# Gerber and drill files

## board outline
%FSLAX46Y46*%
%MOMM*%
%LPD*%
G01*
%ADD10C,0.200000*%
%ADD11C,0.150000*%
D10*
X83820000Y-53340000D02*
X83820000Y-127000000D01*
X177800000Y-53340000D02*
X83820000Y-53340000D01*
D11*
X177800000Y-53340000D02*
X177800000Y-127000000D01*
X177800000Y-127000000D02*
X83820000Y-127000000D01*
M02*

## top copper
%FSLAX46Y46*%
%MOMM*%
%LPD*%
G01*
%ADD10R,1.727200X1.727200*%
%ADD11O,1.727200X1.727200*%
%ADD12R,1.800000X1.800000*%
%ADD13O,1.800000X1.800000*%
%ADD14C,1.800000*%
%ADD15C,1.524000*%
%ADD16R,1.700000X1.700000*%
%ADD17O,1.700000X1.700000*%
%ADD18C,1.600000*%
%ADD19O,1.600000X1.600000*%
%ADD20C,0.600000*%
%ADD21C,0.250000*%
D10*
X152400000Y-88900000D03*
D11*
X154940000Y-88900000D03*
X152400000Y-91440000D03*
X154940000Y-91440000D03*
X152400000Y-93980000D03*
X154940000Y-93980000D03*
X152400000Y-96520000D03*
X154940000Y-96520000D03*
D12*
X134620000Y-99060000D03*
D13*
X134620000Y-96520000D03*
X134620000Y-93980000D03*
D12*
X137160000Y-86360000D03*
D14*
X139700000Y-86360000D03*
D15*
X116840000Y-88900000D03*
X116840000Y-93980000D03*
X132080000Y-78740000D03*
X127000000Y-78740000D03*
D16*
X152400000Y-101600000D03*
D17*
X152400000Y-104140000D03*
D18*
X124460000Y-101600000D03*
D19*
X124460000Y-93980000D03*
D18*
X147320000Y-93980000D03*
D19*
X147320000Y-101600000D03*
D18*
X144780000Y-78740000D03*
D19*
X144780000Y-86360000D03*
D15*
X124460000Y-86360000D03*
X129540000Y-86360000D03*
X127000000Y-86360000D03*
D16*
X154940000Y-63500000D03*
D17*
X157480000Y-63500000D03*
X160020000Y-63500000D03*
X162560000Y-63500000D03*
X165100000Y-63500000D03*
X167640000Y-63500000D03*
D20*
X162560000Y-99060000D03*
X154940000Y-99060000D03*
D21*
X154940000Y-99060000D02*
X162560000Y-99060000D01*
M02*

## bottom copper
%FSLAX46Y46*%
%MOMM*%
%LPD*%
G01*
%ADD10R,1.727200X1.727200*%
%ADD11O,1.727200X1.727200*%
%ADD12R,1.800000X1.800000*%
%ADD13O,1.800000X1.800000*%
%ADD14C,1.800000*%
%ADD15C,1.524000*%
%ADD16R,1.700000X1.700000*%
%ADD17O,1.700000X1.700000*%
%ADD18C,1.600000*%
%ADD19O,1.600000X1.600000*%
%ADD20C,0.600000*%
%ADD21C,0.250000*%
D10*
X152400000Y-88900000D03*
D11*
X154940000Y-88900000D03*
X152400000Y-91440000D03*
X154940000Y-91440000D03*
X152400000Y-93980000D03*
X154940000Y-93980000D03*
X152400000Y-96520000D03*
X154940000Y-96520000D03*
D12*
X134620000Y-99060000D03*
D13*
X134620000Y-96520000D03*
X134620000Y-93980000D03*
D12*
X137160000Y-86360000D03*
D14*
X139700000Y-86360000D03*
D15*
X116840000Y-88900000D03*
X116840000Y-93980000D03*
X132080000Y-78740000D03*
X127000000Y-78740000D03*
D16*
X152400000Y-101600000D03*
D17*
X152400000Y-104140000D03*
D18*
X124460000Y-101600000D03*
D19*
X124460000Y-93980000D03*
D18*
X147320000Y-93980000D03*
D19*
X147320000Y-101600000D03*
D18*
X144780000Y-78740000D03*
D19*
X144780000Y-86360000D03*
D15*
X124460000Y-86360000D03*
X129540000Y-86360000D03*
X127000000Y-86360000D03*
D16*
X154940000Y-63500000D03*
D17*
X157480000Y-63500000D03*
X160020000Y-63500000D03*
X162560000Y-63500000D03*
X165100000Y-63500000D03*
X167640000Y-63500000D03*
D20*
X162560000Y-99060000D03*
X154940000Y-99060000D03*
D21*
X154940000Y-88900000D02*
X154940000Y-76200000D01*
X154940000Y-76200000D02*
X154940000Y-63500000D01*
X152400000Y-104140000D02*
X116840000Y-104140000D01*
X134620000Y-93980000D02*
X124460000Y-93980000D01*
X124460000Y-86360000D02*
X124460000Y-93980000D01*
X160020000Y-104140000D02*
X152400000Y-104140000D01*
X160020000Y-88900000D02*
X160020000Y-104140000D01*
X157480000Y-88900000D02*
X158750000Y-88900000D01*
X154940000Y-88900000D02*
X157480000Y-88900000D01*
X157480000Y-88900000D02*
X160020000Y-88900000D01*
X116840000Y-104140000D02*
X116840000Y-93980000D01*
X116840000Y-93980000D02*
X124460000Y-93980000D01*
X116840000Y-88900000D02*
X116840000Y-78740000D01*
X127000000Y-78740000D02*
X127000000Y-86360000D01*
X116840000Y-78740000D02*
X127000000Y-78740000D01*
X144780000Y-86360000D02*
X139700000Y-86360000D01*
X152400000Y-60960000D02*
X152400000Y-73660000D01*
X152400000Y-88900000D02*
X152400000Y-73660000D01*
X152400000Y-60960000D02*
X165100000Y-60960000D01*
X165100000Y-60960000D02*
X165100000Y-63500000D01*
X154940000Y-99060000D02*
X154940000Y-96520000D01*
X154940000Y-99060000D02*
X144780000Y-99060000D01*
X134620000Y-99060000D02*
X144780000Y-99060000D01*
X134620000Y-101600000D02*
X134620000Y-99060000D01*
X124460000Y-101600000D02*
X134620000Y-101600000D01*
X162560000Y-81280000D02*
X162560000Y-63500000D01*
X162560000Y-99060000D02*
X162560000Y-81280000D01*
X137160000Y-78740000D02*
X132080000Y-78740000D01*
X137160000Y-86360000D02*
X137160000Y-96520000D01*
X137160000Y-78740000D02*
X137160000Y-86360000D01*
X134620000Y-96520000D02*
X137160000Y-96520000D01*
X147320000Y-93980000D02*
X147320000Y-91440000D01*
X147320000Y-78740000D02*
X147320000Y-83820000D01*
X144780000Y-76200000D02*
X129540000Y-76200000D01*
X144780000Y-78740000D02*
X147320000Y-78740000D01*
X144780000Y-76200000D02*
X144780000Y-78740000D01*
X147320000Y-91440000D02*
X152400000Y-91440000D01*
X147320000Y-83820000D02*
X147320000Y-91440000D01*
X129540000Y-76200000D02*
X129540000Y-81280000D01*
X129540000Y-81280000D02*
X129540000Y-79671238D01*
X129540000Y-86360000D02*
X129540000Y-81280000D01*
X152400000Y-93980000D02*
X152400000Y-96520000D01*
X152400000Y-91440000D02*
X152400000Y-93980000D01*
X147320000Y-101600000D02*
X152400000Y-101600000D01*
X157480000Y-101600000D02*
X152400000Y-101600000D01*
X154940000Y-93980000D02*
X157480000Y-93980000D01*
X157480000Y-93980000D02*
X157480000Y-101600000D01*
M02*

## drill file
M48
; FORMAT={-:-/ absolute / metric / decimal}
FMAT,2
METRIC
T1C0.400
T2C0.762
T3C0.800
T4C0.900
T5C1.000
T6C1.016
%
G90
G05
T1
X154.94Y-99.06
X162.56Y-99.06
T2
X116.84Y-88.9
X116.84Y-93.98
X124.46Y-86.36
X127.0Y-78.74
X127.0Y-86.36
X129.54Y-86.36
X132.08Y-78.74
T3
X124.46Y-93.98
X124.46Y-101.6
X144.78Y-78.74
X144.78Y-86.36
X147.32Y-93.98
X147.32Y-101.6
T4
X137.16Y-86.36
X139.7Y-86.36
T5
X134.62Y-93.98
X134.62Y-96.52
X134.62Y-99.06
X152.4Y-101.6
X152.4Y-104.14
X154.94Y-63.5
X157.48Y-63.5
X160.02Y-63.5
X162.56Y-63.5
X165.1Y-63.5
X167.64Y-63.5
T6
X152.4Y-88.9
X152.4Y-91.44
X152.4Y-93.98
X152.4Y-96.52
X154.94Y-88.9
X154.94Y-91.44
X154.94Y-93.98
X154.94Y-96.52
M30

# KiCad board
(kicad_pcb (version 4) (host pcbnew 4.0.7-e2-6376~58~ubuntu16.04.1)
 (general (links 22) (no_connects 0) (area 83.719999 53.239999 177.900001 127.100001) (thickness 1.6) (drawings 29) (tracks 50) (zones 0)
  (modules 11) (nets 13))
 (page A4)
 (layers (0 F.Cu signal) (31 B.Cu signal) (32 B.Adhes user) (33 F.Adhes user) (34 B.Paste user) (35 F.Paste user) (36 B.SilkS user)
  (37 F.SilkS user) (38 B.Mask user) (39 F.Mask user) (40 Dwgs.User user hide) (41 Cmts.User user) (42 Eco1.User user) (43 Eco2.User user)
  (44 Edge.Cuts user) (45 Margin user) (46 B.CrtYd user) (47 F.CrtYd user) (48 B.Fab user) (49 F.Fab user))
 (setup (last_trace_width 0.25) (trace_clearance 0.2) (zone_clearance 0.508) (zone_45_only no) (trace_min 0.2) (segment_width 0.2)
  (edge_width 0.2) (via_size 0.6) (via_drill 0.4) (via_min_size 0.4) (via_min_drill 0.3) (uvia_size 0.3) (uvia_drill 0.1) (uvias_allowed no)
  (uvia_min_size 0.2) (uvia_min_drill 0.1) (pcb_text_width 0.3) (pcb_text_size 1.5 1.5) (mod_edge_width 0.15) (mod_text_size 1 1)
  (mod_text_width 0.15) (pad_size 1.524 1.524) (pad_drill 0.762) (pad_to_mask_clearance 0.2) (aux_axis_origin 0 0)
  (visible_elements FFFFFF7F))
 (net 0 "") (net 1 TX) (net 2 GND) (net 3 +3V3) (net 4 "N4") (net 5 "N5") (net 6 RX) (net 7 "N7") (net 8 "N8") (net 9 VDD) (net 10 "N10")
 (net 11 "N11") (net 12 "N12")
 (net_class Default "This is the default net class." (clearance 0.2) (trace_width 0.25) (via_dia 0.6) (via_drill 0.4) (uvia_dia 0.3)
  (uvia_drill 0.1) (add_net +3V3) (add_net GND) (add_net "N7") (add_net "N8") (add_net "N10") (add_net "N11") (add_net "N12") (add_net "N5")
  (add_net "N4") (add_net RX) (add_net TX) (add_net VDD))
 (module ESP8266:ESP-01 (layer F.Cu) (at 152.4 88.9)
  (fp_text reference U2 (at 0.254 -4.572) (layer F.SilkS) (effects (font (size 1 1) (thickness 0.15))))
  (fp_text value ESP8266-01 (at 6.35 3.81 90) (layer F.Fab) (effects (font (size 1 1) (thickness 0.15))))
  (pad 1 thru_hole rect (at 0 0) (size 1.7272 1.7272) (drill 1.016) (layers *.Cu *.Mask F.SilkS) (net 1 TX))
  (pad 2 thru_hole oval (at 2.54 0) (size 1.7272 1.7272) (drill 1.016) (layers *.Cu *.Mask F.SilkS) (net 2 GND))
  (pad 3 thru_hole oval (at 0 2.54) (size 1.7272 1.7272) (drill 1.016) (layers *.Cu *.Mask F.SilkS) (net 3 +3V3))
  (pad 4 thru_hole oval (at 2.54 2.54) (size 1.7272 1.7272) (drill 1.016) (layers *.Cu *.Mask F.SilkS) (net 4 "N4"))
  (pad 5 thru_hole oval (at 0 5.08) (size 1.7272 1.7272) (drill 1.016) (layers *.Cu *.Mask F.SilkS) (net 3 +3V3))
  (pad 6 thru_hole oval (at 2.54 5.08) (size 1.7272 1.7272) (drill 1.016) (layers *.Cu *.Mask F.SilkS) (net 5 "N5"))
  (pad 7 thru_hole oval (at 0 7.62) (size 1.7272 1.7272) (drill 1.016) (layers *.Cu *.Mask F.SilkS) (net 3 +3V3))
  (pad 8 thru_hole oval (at 2.54 7.62) (size 1.7272 1.7272) (drill 1.016) (layers *.Cu *.Mask F.SilkS) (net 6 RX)))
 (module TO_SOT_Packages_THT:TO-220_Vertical (layer F.Cu) (at 134.62 99.06 90)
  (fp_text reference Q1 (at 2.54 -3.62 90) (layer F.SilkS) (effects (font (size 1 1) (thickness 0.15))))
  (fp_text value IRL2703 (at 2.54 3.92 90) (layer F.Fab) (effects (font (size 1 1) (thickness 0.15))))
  (pad 1 thru_hole rect (at 0 0 90) (size 1.8 1.8) (drill 1) (layers *.Cu *.Mask) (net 6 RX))
  (pad 2 thru_hole oval (at 2.54 0 90) (size 1.8 1.8) (drill 1) (layers *.Cu *.Mask) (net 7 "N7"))
  (pad 3 thru_hole oval (at 5.08 0 90) (size 1.8 1.8) (drill 1) (layers *.Cu *.Mask) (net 2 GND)))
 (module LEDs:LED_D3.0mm (layer F.Cu) (at 137.16 86.36)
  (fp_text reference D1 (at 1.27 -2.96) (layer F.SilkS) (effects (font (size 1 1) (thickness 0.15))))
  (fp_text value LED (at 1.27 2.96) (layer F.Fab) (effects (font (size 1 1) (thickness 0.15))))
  (pad 1 thru_hole rect (at 0 0) (size 1.8 1.8) (drill 0.9) (layers *.Cu *.Mask) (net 7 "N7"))
  (pad 2 thru_hole circle (at 2.54 0) (size 1.8 1.8) (drill 0.9) (layers *.Cu *.Mask) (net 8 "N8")))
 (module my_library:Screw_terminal (layer F.Cu) (at 116.84 91.44 270)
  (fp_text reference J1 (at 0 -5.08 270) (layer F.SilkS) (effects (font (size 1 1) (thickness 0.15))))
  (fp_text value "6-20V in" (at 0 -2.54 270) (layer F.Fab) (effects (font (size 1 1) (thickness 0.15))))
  (pad 1 thru_hole circle (at -2.54 0 270) (size 1.524 1.524) (drill 0.762) (layers *.Cu *.Mask F.SilkS) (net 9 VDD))
  (pad 2 thru_hole circle (at 2.54 0 270) (size 1.524 1.524) (drill 0.762) (layers *.Cu *.Mask F.SilkS) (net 2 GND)))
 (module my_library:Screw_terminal (layer F.Cu) (at 129.54 78.74 180)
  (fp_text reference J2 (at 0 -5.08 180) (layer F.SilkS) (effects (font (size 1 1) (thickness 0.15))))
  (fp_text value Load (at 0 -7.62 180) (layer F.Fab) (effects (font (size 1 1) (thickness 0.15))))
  (pad 1 thru_hole circle (at -2.54 0 180) (size 1.524 1.524) (drill 0.762) (layers *.Cu *.Mask F.SilkS) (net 7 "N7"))
  (pad 2 thru_hole circle (at 2.54 0 180) (size 1.524 1.524) (drill 0.762) (layers *.Cu *.Mask F.SilkS) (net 9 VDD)))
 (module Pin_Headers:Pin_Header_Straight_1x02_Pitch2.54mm (layer F.Cu) (at 152.4 101.6)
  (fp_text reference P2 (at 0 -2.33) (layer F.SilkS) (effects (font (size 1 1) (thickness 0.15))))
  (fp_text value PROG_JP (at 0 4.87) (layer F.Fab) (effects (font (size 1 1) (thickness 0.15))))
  (pad 1 thru_hole rect (at 0 0) (size 1.7 1.7) (drill 1) (layers *.Cu *.Mask) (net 5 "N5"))
  (pad 2 thru_hole oval (at 0 2.54) (size 1.7 1.7) (drill 1) (layers *.Cu *.Mask) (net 2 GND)))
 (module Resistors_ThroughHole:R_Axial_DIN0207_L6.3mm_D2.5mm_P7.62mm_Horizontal (layer F.Cu) (at 124.46 101.6 90)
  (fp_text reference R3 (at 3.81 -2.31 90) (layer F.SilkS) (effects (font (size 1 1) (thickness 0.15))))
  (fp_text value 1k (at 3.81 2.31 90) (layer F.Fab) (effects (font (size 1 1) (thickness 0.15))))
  (pad 1 thru_hole circle (at 0 0 90) (size 1.6 1.6) (drill 0.8) (layers *.Cu *.Mask) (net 6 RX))
  (pad 2 thru_hole oval (at 7.62 0 90) (size 1.6 1.6) (drill 0.8) (layers *.Cu *.Mask) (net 2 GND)))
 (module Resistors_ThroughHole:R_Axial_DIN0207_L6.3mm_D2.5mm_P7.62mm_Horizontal (layer F.Cu) (at 147.32 93.98 270)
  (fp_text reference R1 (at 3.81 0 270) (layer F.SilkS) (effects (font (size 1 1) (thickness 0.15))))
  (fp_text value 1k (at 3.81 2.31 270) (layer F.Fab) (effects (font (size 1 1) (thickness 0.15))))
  (pad 1 thru_hole circle (at 0 0 270) (size 1.6 1.6) (drill 0.8) (layers *.Cu *.Mask) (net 3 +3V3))
  (pad 2 thru_hole oval (at 7.62 0 270) (size 1.6 1.6) (drill 0.8) (layers *.Cu *.Mask) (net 5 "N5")))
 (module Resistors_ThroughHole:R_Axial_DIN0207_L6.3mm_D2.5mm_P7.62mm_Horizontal (layer F.Cu) (at 144.78 78.74 270)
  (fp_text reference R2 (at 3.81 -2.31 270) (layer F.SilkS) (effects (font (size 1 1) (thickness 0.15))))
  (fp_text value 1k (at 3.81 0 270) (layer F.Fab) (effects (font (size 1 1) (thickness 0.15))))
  (pad 1 thru_hole circle (at 0 0 270) (size 1.6 1.6) (drill 0.8) (layers *.Cu *.Mask) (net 3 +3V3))
  (pad 2 thru_hole oval (at 7.62 0 270) (size 1.6 1.6) (drill 0.8) (layers *.Cu *.Mask) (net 8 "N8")))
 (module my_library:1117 (layer F.Cu) (at 127 86.36 180)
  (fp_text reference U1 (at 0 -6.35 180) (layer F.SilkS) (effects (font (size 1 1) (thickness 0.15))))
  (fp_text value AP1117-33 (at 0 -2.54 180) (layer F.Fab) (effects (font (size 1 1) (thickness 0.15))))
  (pad 1 thru_hole circle (at 2.54 0 180) (size 1.524 1.524) (drill 0.762) (layers *.Cu *.Mask F.SilkS) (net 2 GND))
  (pad 2 thru_hole circle (at -2.54 0 180) (size 1.524 1.524) (drill 0.762) (layers *.Cu *.Mask F.SilkS) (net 3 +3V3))
  (pad 3 thru_hole circle (at 0 0 180) (size 1.524 1.524) (drill 0.762) (layers *.Cu *.Mask F.SilkS) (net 9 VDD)))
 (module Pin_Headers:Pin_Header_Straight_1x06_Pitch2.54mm (layer F.Cu) (at 154.94 63.5 90)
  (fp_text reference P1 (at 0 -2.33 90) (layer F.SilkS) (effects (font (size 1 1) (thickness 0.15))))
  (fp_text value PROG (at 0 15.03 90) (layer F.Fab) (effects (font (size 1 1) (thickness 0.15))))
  (pad 1 thru_hole rect (at 0 0 90) (size 1.7 1.7) (drill 1) (layers *.Cu *.Mask) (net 2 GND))
  (pad 2 thru_hole oval (at 0 2.54 90) (size 1.7 1.7) (drill 1) (layers *.Cu *.Mask) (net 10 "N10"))
  (pad 3 thru_hole oval (at 0 5.08 90) (size 1.7 1.7) (drill 1) (layers *.Cu *.Mask) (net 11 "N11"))
  (pad 4 thru_hole oval (at 0 7.62 90) (size 1.7 1.7) (drill 1) (layers *.Cu *.Mask) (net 6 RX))
  (pad 5 thru_hole oval (at 0 10.16 90) (size 1.7 1.7) (drill 1) (layers *.Cu *.Mask) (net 1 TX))
  (pad 6 thru_hole oval (at 0 12.7 90) (size 1.7 1.7) (drill 1) (layers *.Cu *.Mask) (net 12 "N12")))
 (gr_line (start 83.82 53.34) (end 83.82 127) (layer Edge.Cuts) (width 0.2))
 (gr_line (start 177.8 53.34) (end 83.82 53.34) (layer Edge.Cuts) (width 0.2))
 (gr_line (start 177.8 53.34) (end 177.8 127) (angle 90) (layer Edge.Cuts) (width 0.15))
 (gr_line (start 177.8 127) (end 83.82 127) (angle 90) (layer Edge.Cuts) (width 0.15))
 (segment (start 154.94 88.9) (end 154.94 76.2) (width 0.25) (layer B.Cu) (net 2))
 (segment (start 154.94 76.2) (end 154.94 63.5) (width 0.25) (layer B.Cu) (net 2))
 (segment (start 152.4 104.14) (end 116.84 104.14) (width 0.25) (layer B.Cu) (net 2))
 (segment (start 134.62 93.98) (end 124.46 93.98) (width 0.25) (layer B.Cu) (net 2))
 (segment (start 124.46 86.36) (end 124.46 93.98) (width 0.25) (layer B.Cu) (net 2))
 (segment (start 160.02 104.14) (end 152.4 104.14) (width 0.25) (layer B.Cu) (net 2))
 (segment (start 160.02 88.9) (end 160.02 104.14) (width 0.25) (layer B.Cu) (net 2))
 (segment (start 157.48 88.9) (end 158.75 88.9) (width 0.25) (layer B.Cu) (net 2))
 (segment (start 154.94 88.9) (end 157.48 88.9) (width 0.25) (layer B.Cu) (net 2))
 (segment (start 157.48 88.9) (end 160.02 88.9) (width 0.25) (layer B.Cu) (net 2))
 (segment (start 116.84 104.14) (end 116.84 93.98) (width 0.25) (layer B.Cu) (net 2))
 (segment (start 116.84 93.98) (end 124.46 93.98) (width 0.25) (layer B.Cu) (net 2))
 (segment (start 116.84 88.9) (end 116.84 78.74) (width 0.25) (layer B.Cu) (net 9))
 (segment (start 127 78.74) (end 127 86.36) (width 0.25) (layer B.Cu) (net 9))
 (segment (start 116.84 78.74) (end 127 78.74) (width 0.25) (layer B.Cu) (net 9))
 (segment (start 144.78 86.36) (end 139.7 86.36) (width 0.25) (layer B.Cu) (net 8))
 (segment (start 152.4 60.96) (end 152.4 73.66) (width 0.25) (layer B.Cu) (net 1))
 (segment (start 152.4 88.9) (end 152.4 73.66) (width 0.25) (layer B.Cu) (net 1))
 (segment (start 152.4 60.96) (end 165.1 60.96) (width 0.25) (layer B.Cu) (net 1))
 (segment (start 165.1 60.96) (end 165.1 63.5) (width 0.25) (layer B.Cu) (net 1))
 (segment (start 154.94 99.06) (end 154.94 96.52) (width 0.25) (layer B.Cu) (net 6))
 (segment (start 154.94 99.06) (end 144.78 99.06) (width 0.25) (layer B.Cu) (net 6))
 (segment (start 134.62 99.06) (end 144.78 99.06) (width 0.25) (layer B.Cu) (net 6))
 (segment (start 134.62 101.6) (end 134.62 99.06) (width 0.25) (layer B.Cu) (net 6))
 (segment (start 124.46 101.6) (end 134.62 101.6) (width 0.25) (layer B.Cu) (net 6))
 (segment (start 162.56 81.28) (end 162.56 63.5) (width 0.25) (layer B.Cu) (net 6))
 (segment (start 162.56 99.06) (end 162.56 81.28) (width 0.25) (layer B.Cu) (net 6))
 (segment (start 154.94 99.06) (end 162.56 99.06) (width 0.25) (layer F.Cu) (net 6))
 (via (at 162.56 99.06) (size 0.6) (drill 0.4) (layers F.Cu B.Cu) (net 6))
 (via (at 154.94 99.06) (size 0.6) (drill 0.4) (layers F.Cu B.Cu) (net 6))
 (segment (start 137.16 78.74) (end 132.08 78.74) (width 0.25) (layer B.Cu) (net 7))
 (segment (start 137.16 86.36) (end 137.16 96.52) (width 0.25) (layer B.Cu) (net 7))
 (segment (start 137.16 78.74) (end 137.16 86.36) (width 0.25) (layer B.Cu) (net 7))
 (segment (start 134.62 96.52) (end 137.16 96.52) (width 0.25) (layer B.Cu) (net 7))
 (segment (start 147.32 93.98) (end 147.32 91.44) (width 0.25) (layer B.Cu) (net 3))
 (segment (start 147.32 78.74) (end 147.32 83.82) (width 0.25) (layer B.Cu) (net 3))
 (segment (start 144.78 76.2) (end 129.54 76.2) (width 0.25) (layer B.Cu) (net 3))
 (segment (start 144.78 78.74) (end 147.32 78.74) (width 0.25) (layer B.Cu) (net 3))
 (segment (start 144.78 76.2) (end 144.78 78.74) (width 0.25) (layer B.Cu) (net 3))
 (segment (start 147.32 91.44) (end 152.4 91.44) (width 0.25) (layer B.Cu) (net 3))
 (segment (start 147.32 83.82) (end 147.32 91.44) (width 0.25) (layer B.Cu) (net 3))
 (segment (start 129.54 76.2) (end 129.54 81.28) (width 0.25) (layer B.Cu) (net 3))
 (segment (start 129.54 81.28) (end 129.54 79.671238) (width 0.25) (layer B.Cu) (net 3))
 (segment (start 129.54 86.36) (end 129.54 81.28) (width 0.25) (layer B.Cu) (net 3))
 (segment (start 152.4 93.98) (end 152.4 96.52) (width 0.25) (layer B.Cu) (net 3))
 (segment (start 152.4 91.44) (end 152.4 93.98) (width 0.25) (layer B.Cu) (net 3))
 (segment (start 147.32 101.6) (end 152.4 101.6) (width 0.25) (layer B.Cu) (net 5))
 (segment (start 157.48 101.6) (end 152.4 101.6) (width 0.25) (layer B.Cu) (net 5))
 (segment (start 154.94 93.98) (end 157.48 93.98) (width 0.25) (layer B.Cu) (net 5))
 (segment (start 157.48 93.98) (end 157.48 101.6) (width 0.25) (layer B.Cu) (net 5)))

